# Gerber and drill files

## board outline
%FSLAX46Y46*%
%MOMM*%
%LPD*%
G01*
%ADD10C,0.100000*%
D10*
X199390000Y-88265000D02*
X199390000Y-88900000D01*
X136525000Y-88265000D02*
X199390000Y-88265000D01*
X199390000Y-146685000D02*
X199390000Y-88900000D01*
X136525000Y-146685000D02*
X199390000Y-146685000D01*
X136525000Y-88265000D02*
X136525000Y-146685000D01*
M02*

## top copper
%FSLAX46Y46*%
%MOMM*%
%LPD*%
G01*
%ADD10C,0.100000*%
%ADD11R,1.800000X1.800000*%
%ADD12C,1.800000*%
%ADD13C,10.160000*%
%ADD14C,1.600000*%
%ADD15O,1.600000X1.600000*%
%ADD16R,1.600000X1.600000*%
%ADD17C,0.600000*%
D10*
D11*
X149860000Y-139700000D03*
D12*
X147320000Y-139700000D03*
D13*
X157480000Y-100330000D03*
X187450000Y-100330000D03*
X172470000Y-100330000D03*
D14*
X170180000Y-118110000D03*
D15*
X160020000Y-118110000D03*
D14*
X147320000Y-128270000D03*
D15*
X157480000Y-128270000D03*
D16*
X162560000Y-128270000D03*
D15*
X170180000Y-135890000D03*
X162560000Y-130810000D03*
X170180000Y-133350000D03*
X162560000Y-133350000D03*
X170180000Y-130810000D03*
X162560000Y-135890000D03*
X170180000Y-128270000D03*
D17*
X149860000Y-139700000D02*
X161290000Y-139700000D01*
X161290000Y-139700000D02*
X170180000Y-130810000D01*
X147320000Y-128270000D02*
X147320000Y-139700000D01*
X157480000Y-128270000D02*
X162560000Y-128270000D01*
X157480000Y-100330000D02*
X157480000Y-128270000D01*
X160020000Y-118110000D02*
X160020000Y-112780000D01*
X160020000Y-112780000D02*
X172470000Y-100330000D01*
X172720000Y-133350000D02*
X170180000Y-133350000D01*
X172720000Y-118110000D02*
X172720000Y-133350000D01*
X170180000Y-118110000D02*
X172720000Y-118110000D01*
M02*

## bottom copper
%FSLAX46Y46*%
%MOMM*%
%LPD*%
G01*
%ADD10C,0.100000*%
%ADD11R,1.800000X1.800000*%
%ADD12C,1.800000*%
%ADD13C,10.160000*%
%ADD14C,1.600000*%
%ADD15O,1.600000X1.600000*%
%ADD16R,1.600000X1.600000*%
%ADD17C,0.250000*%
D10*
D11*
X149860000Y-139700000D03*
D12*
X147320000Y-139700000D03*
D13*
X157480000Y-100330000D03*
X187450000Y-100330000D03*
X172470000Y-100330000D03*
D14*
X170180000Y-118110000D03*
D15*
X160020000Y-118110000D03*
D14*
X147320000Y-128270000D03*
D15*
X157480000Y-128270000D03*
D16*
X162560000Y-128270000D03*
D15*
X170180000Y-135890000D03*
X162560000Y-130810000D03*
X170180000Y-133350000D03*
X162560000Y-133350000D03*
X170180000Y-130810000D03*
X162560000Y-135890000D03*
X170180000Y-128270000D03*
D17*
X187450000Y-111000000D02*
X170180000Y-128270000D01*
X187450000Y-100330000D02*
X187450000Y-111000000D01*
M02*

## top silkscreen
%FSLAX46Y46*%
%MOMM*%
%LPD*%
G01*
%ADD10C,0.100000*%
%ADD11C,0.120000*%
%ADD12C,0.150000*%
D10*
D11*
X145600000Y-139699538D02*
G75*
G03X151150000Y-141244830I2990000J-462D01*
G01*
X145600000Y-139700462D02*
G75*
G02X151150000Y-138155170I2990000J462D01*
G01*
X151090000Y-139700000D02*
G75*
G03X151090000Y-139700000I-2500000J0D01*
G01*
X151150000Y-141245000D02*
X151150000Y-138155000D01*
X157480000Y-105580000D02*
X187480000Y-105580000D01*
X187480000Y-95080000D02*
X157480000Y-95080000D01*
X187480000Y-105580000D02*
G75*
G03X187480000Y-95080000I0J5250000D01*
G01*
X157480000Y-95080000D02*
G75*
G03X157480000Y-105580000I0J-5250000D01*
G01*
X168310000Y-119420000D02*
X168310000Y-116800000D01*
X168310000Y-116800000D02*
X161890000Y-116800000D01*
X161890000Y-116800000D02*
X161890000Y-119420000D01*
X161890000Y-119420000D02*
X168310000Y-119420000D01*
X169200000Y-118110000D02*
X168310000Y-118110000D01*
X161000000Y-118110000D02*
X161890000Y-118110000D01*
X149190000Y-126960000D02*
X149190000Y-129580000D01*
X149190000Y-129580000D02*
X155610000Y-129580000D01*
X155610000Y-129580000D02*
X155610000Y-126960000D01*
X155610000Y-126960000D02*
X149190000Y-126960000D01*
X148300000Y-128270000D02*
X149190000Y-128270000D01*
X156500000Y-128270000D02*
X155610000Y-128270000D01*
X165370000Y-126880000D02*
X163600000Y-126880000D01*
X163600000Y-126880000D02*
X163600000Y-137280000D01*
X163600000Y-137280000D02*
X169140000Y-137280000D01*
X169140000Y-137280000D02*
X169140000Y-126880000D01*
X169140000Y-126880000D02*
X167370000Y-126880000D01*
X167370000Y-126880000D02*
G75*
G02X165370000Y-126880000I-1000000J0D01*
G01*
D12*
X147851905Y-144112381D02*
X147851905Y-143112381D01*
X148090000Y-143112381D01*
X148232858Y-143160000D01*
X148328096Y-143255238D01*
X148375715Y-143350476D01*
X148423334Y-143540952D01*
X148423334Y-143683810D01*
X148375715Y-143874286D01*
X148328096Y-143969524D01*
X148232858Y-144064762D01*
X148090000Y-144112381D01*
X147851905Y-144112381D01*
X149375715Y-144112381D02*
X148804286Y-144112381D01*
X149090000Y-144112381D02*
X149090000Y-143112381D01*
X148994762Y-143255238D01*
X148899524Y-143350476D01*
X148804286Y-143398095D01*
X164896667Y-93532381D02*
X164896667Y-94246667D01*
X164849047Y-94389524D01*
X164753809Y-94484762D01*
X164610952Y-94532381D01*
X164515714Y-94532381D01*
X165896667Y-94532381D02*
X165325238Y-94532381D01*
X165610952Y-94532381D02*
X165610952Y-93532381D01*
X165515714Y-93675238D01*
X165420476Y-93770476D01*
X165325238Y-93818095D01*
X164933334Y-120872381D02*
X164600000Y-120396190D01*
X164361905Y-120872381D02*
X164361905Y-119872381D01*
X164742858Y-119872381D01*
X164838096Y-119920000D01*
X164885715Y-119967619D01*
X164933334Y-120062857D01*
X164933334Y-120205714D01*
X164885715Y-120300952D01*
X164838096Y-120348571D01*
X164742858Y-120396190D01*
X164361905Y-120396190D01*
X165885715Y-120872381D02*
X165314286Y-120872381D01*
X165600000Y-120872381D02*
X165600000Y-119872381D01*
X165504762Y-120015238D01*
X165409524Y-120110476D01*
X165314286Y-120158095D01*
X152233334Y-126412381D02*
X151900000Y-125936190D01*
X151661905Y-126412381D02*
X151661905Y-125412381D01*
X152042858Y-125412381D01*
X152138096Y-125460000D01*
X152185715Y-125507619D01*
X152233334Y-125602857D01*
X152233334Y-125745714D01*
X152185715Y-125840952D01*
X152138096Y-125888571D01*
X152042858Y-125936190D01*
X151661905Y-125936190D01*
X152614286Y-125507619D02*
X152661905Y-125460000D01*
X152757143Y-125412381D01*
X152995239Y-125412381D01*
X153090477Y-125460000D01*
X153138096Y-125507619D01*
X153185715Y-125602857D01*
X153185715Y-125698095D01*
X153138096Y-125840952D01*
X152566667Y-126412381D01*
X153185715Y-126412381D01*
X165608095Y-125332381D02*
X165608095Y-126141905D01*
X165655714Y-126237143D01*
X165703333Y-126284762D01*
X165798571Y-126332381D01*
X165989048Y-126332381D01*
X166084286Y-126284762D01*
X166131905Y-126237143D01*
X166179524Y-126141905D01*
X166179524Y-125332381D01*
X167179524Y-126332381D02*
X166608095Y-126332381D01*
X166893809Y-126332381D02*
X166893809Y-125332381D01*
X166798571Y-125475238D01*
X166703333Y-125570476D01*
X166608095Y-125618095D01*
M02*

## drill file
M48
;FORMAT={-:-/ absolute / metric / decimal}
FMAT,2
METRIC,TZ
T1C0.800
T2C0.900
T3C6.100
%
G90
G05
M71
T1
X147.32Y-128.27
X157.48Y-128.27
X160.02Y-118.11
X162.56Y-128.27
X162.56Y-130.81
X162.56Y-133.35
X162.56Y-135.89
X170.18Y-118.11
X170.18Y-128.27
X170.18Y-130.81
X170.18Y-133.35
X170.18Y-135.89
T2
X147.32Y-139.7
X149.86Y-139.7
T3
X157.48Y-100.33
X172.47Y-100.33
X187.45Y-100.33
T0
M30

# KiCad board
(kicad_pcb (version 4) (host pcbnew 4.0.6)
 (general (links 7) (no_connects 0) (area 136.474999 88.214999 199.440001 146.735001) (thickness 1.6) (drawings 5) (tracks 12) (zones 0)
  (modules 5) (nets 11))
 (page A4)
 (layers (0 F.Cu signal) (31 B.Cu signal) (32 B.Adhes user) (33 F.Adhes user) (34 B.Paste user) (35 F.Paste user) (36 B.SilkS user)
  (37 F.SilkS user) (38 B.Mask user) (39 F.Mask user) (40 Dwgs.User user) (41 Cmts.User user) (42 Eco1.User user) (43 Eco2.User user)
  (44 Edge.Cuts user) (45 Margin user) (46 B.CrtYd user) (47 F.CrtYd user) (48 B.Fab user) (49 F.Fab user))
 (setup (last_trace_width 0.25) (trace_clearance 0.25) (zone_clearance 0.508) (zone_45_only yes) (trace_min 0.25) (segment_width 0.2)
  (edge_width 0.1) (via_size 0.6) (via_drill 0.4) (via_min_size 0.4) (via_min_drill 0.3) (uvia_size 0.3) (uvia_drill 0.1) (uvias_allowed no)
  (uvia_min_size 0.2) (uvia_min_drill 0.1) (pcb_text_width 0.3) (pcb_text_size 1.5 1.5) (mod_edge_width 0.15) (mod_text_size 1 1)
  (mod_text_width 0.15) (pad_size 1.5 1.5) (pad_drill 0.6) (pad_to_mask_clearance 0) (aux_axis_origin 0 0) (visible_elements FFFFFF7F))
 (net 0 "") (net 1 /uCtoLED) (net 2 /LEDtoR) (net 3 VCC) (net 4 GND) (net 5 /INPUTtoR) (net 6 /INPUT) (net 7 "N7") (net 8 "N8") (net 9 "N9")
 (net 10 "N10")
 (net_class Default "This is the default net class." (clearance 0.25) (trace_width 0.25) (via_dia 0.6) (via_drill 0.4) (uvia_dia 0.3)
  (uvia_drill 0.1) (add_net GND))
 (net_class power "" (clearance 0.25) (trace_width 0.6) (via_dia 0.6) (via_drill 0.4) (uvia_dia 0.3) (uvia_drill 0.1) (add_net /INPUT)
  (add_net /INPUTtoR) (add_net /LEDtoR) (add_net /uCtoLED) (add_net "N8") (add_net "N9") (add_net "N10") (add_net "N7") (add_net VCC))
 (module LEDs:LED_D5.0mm (layer F.Cu) (at 149.86 139.7 180)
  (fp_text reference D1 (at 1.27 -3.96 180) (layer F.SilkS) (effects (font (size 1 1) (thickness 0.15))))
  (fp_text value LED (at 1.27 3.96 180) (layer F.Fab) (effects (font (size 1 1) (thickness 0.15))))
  (fp_arc (start 1.27 0) (end -1.29 -1.54483) (angle 148.9) (layer F.SilkS) (width 0.12))
  (fp_arc (start 1.27 0) (end -1.29 1.54483) (angle -148.9) (layer F.SilkS) (width 0.12))
  (fp_circle (center 1.27 0) (end 3.77 0) (layer F.SilkS) (width 0.12))
  (fp_line (start -1.29 -1.545) (end -1.29 1.545) (layer F.SilkS) (width 0.12))
  (pad 1 thru_hole rect (at 0 0 180) (size 1.8 1.8) (drill 0.9) (layers *.Cu *.Mask) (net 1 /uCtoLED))
  (pad 2 thru_hole circle (at 2.54 0 180) (size 1.8 1.8) (drill 0.9) (layers *.Cu *.Mask) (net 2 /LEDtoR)))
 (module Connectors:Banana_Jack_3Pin (layer F.Cu) (at 157.48 100.33)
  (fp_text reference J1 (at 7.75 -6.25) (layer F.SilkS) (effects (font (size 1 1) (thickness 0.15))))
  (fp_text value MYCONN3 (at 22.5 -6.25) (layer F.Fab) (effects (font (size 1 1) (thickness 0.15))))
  (fp_line (start 0 5.25) (end 30 5.25) (layer F.SilkS) (width 0.12))
  (fp_line (start 30 -5.25) (end 0 -5.25) (layer F.SilkS) (width 0.12))
  (fp_arc (start 30 0) (end 30 -5.25) (angle 180) (layer F.SilkS) (width 0.12))
  (fp_arc (start 0 0) (end 0 5.25) (angle 180) (layer F.SilkS) (width 0.12))
  (pad 1 thru_hole circle (at 0 0) (size 10.16 10.16) (drill 6.1) (layers *.Cu *.Mask) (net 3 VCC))
  (pad 3 thru_hole circle (at 29.97 0) (size 10.16 10.16) (drill 6.1) (layers *.Cu *.Mask) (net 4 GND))
  (pad 2 thru_hole circle (at 14.99 0) (size 10.16 10.16) (drill 6.1) (layers *.Cu *.Mask) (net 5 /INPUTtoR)))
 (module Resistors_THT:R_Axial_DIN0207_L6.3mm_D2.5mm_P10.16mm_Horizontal (layer F.Cu) (at 170.18 118.11 180)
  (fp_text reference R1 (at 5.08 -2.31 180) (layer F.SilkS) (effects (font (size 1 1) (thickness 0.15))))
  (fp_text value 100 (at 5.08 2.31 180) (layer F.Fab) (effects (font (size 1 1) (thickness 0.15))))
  (fp_line (start 1.87 -1.31) (end 1.87 1.31) (layer F.SilkS) (width 0.12))
  (fp_line (start 1.87 1.31) (end 8.29 1.31) (layer F.SilkS) (width 0.12))
  (fp_line (start 8.29 1.31) (end 8.29 -1.31) (layer F.SilkS) (width 0.12))
  (fp_line (start 8.29 -1.31) (end 1.87 -1.31) (layer F.SilkS) (width 0.12))
  (fp_line (start 0.98 0) (end 1.87 0) (layer F.SilkS) (width 0.12))
  (fp_line (start 9.18 0) (end 8.29 0) (layer F.SilkS) (width 0.12))
  (pad 1 thru_hole circle (at 0 0 180) (size 1.6 1.6) (drill 0.8) (layers *.Cu *.Mask) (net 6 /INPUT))
  (pad 2 thru_hole oval (at 10.16 0 180) (size 1.6 1.6) (drill 0.8) (layers *.Cu *.Mask) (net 5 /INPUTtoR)))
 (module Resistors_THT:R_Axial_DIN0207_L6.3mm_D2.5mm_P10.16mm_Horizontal (layer F.Cu) (at 147.32 128.27)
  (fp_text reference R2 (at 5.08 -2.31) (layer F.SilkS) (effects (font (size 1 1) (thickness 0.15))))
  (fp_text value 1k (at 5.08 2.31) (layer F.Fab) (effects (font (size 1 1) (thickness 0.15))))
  (fp_line (start 1.87 -1.31) (end 1.87 1.31) (layer F.SilkS) (width 0.12))
  (fp_line (start 1.87 1.31) (end 8.29 1.31) (layer F.SilkS) (width 0.12))
  (fp_line (start 8.29 1.31) (end 8.29 -1.31) (layer F.SilkS) (width 0.12))
  (fp_line (start 8.29 -1.31) (end 1.87 -1.31) (layer F.SilkS) (width 0.12))
  (fp_line (start 0.98 0) (end 1.87 0) (layer F.SilkS) (width 0.12))
  (fp_line (start 9.18 0) (end 8.29 0) (layer F.SilkS) (width 0.12))
  (pad 1 thru_hole circle (at 0 0) (size 1.6 1.6) (drill 0.8) (layers *.Cu *.Mask) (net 2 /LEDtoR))
  (pad 2 thru_hole oval (at 10.16 0) (size 1.6 1.6) (drill 0.8) (layers *.Cu *.Mask) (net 3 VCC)))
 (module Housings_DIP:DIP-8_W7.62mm (layer F.Cu) (at 162.56 128.27)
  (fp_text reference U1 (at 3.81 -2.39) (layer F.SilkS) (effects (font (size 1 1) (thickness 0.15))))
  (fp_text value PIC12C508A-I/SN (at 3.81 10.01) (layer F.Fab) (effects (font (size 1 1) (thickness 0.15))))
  (fp_line (start 2.81 -1.39) (end 1.04 -1.39) (layer F.SilkS) (width 0.12))
  (fp_line (start 1.04 -1.39) (end 1.04 9.01) (layer F.SilkS) (width 0.12))
  (fp_line (start 1.04 9.01) (end 6.58 9.01) (layer F.SilkS) (width 0.12))
  (fp_line (start 6.58 9.01) (end 6.58 -1.39) (layer F.SilkS) (width 0.12))
  (fp_line (start 6.58 -1.39) (end 4.81 -1.39) (layer F.SilkS) (width 0.12))
  (fp_arc (start 3.81 -1.39) (end 2.81 -1.39) (angle -180) (layer F.SilkS) (width 0.12))
  (pad 1 thru_hole rect (at 0 0) (size 1.6 1.6) (drill 0.8) (layers *.Cu *.Mask) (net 3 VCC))
  (pad 5 thru_hole oval (at 7.62 7.62) (size 1.6 1.6) (drill 0.8) (layers *.Cu *.Mask) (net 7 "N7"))
  (pad 2 thru_hole oval (at 0 2.54) (size 1.6 1.6) (drill 0.8) (layers *.Cu *.Mask) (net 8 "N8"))
  (pad 6 thru_hole oval (at 7.62 5.08) (size 1.6 1.6) (drill 0.8) (layers *.Cu *.Mask) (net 6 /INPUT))
  (pad 3 thru_hole oval (at 0 5.08) (size 1.6 1.6) (drill 0.8) (layers *.Cu *.Mask) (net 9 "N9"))
  (pad 7 thru_hole oval (at 7.62 2.54) (size 1.6 1.6) (drill 0.8) (layers *.Cu *.Mask) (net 1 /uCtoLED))
  (pad 4 thru_hole oval (at 0 7.62) (size 1.6 1.6) (drill 0.8) (layers *.Cu *.Mask) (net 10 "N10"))
  (pad 8 thru_hole oval (at 7.62 0) (size 1.6 1.6) (drill 0.8) (layers *.Cu *.Mask) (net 4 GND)))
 (gr_line (start 199.39 88.265) (end 199.39 88.9) (angle 90) (layer Edge.Cuts) (width 0.1))
 (gr_line (start 136.525 88.265) (end 199.39 88.265) (angle 90) (layer Edge.Cuts) (width 0.1))
 (gr_line (start 199.39 146.685) (end 199.39 88.9) (angle 90) (layer Edge.Cuts) (width 0.1))
 (gr_line (start 136.525 146.685) (end 199.39 146.685) (angle 90) (layer Edge.Cuts) (width 0.1))
 (gr_line (start 136.525 88.265) (end 136.525 146.685) (angle 90) (layer Edge.Cuts) (width 0.1))
 (segment (start 149.86 139.7) (end 161.29 139.7) (width 0.6) (layer F.Cu) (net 1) (status 10))
 (segment (start 161.29 139.7) (end 170.18 130.81) (width 0.6) (layer F.Cu) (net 1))
 (segment (start 147.32 128.27) (end 147.32 139.7) (width 0.6) (layer F.Cu) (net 2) (status 20))
 (segment (start 157.48 128.27) (end 162.56 128.27) (width 0.6) (layer F.Cu) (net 3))
 (segment (start 157.48 100.33) (end 157.48 128.27) (width 0.6) (layer F.Cu) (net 3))
 (segment (start 187.45 111) (end 170.18 128.27) (width 0.25) (layer B.Cu) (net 4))
 (segment (start 187.45 100.33) (end 187.45 111) (width 0.25) (layer B.Cu) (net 4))
 (segment (start 160.02 118.11) (end 160.02 112.78) (width 0.6) (layer F.Cu) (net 5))
 (segment (start 160.02 112.78) (end 172.47 100.33) (width 0.6) (layer F.Cu) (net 5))
 (segment (start 172.72 133.35) (end 170.18 133.35) (width 0.6) (layer F.Cu) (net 6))
 (segment (start 172.72 118.11) (end 172.72 133.35) (width 0.6) (layer F.Cu) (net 6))
 (segment (start 170.18 118.11) (end 172.72 118.11) (width 0.6) (layer F.Cu) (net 6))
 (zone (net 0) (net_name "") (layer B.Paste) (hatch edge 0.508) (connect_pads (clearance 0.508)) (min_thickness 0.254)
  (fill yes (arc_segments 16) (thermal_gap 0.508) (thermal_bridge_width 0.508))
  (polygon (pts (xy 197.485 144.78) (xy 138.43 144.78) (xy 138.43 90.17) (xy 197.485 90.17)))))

